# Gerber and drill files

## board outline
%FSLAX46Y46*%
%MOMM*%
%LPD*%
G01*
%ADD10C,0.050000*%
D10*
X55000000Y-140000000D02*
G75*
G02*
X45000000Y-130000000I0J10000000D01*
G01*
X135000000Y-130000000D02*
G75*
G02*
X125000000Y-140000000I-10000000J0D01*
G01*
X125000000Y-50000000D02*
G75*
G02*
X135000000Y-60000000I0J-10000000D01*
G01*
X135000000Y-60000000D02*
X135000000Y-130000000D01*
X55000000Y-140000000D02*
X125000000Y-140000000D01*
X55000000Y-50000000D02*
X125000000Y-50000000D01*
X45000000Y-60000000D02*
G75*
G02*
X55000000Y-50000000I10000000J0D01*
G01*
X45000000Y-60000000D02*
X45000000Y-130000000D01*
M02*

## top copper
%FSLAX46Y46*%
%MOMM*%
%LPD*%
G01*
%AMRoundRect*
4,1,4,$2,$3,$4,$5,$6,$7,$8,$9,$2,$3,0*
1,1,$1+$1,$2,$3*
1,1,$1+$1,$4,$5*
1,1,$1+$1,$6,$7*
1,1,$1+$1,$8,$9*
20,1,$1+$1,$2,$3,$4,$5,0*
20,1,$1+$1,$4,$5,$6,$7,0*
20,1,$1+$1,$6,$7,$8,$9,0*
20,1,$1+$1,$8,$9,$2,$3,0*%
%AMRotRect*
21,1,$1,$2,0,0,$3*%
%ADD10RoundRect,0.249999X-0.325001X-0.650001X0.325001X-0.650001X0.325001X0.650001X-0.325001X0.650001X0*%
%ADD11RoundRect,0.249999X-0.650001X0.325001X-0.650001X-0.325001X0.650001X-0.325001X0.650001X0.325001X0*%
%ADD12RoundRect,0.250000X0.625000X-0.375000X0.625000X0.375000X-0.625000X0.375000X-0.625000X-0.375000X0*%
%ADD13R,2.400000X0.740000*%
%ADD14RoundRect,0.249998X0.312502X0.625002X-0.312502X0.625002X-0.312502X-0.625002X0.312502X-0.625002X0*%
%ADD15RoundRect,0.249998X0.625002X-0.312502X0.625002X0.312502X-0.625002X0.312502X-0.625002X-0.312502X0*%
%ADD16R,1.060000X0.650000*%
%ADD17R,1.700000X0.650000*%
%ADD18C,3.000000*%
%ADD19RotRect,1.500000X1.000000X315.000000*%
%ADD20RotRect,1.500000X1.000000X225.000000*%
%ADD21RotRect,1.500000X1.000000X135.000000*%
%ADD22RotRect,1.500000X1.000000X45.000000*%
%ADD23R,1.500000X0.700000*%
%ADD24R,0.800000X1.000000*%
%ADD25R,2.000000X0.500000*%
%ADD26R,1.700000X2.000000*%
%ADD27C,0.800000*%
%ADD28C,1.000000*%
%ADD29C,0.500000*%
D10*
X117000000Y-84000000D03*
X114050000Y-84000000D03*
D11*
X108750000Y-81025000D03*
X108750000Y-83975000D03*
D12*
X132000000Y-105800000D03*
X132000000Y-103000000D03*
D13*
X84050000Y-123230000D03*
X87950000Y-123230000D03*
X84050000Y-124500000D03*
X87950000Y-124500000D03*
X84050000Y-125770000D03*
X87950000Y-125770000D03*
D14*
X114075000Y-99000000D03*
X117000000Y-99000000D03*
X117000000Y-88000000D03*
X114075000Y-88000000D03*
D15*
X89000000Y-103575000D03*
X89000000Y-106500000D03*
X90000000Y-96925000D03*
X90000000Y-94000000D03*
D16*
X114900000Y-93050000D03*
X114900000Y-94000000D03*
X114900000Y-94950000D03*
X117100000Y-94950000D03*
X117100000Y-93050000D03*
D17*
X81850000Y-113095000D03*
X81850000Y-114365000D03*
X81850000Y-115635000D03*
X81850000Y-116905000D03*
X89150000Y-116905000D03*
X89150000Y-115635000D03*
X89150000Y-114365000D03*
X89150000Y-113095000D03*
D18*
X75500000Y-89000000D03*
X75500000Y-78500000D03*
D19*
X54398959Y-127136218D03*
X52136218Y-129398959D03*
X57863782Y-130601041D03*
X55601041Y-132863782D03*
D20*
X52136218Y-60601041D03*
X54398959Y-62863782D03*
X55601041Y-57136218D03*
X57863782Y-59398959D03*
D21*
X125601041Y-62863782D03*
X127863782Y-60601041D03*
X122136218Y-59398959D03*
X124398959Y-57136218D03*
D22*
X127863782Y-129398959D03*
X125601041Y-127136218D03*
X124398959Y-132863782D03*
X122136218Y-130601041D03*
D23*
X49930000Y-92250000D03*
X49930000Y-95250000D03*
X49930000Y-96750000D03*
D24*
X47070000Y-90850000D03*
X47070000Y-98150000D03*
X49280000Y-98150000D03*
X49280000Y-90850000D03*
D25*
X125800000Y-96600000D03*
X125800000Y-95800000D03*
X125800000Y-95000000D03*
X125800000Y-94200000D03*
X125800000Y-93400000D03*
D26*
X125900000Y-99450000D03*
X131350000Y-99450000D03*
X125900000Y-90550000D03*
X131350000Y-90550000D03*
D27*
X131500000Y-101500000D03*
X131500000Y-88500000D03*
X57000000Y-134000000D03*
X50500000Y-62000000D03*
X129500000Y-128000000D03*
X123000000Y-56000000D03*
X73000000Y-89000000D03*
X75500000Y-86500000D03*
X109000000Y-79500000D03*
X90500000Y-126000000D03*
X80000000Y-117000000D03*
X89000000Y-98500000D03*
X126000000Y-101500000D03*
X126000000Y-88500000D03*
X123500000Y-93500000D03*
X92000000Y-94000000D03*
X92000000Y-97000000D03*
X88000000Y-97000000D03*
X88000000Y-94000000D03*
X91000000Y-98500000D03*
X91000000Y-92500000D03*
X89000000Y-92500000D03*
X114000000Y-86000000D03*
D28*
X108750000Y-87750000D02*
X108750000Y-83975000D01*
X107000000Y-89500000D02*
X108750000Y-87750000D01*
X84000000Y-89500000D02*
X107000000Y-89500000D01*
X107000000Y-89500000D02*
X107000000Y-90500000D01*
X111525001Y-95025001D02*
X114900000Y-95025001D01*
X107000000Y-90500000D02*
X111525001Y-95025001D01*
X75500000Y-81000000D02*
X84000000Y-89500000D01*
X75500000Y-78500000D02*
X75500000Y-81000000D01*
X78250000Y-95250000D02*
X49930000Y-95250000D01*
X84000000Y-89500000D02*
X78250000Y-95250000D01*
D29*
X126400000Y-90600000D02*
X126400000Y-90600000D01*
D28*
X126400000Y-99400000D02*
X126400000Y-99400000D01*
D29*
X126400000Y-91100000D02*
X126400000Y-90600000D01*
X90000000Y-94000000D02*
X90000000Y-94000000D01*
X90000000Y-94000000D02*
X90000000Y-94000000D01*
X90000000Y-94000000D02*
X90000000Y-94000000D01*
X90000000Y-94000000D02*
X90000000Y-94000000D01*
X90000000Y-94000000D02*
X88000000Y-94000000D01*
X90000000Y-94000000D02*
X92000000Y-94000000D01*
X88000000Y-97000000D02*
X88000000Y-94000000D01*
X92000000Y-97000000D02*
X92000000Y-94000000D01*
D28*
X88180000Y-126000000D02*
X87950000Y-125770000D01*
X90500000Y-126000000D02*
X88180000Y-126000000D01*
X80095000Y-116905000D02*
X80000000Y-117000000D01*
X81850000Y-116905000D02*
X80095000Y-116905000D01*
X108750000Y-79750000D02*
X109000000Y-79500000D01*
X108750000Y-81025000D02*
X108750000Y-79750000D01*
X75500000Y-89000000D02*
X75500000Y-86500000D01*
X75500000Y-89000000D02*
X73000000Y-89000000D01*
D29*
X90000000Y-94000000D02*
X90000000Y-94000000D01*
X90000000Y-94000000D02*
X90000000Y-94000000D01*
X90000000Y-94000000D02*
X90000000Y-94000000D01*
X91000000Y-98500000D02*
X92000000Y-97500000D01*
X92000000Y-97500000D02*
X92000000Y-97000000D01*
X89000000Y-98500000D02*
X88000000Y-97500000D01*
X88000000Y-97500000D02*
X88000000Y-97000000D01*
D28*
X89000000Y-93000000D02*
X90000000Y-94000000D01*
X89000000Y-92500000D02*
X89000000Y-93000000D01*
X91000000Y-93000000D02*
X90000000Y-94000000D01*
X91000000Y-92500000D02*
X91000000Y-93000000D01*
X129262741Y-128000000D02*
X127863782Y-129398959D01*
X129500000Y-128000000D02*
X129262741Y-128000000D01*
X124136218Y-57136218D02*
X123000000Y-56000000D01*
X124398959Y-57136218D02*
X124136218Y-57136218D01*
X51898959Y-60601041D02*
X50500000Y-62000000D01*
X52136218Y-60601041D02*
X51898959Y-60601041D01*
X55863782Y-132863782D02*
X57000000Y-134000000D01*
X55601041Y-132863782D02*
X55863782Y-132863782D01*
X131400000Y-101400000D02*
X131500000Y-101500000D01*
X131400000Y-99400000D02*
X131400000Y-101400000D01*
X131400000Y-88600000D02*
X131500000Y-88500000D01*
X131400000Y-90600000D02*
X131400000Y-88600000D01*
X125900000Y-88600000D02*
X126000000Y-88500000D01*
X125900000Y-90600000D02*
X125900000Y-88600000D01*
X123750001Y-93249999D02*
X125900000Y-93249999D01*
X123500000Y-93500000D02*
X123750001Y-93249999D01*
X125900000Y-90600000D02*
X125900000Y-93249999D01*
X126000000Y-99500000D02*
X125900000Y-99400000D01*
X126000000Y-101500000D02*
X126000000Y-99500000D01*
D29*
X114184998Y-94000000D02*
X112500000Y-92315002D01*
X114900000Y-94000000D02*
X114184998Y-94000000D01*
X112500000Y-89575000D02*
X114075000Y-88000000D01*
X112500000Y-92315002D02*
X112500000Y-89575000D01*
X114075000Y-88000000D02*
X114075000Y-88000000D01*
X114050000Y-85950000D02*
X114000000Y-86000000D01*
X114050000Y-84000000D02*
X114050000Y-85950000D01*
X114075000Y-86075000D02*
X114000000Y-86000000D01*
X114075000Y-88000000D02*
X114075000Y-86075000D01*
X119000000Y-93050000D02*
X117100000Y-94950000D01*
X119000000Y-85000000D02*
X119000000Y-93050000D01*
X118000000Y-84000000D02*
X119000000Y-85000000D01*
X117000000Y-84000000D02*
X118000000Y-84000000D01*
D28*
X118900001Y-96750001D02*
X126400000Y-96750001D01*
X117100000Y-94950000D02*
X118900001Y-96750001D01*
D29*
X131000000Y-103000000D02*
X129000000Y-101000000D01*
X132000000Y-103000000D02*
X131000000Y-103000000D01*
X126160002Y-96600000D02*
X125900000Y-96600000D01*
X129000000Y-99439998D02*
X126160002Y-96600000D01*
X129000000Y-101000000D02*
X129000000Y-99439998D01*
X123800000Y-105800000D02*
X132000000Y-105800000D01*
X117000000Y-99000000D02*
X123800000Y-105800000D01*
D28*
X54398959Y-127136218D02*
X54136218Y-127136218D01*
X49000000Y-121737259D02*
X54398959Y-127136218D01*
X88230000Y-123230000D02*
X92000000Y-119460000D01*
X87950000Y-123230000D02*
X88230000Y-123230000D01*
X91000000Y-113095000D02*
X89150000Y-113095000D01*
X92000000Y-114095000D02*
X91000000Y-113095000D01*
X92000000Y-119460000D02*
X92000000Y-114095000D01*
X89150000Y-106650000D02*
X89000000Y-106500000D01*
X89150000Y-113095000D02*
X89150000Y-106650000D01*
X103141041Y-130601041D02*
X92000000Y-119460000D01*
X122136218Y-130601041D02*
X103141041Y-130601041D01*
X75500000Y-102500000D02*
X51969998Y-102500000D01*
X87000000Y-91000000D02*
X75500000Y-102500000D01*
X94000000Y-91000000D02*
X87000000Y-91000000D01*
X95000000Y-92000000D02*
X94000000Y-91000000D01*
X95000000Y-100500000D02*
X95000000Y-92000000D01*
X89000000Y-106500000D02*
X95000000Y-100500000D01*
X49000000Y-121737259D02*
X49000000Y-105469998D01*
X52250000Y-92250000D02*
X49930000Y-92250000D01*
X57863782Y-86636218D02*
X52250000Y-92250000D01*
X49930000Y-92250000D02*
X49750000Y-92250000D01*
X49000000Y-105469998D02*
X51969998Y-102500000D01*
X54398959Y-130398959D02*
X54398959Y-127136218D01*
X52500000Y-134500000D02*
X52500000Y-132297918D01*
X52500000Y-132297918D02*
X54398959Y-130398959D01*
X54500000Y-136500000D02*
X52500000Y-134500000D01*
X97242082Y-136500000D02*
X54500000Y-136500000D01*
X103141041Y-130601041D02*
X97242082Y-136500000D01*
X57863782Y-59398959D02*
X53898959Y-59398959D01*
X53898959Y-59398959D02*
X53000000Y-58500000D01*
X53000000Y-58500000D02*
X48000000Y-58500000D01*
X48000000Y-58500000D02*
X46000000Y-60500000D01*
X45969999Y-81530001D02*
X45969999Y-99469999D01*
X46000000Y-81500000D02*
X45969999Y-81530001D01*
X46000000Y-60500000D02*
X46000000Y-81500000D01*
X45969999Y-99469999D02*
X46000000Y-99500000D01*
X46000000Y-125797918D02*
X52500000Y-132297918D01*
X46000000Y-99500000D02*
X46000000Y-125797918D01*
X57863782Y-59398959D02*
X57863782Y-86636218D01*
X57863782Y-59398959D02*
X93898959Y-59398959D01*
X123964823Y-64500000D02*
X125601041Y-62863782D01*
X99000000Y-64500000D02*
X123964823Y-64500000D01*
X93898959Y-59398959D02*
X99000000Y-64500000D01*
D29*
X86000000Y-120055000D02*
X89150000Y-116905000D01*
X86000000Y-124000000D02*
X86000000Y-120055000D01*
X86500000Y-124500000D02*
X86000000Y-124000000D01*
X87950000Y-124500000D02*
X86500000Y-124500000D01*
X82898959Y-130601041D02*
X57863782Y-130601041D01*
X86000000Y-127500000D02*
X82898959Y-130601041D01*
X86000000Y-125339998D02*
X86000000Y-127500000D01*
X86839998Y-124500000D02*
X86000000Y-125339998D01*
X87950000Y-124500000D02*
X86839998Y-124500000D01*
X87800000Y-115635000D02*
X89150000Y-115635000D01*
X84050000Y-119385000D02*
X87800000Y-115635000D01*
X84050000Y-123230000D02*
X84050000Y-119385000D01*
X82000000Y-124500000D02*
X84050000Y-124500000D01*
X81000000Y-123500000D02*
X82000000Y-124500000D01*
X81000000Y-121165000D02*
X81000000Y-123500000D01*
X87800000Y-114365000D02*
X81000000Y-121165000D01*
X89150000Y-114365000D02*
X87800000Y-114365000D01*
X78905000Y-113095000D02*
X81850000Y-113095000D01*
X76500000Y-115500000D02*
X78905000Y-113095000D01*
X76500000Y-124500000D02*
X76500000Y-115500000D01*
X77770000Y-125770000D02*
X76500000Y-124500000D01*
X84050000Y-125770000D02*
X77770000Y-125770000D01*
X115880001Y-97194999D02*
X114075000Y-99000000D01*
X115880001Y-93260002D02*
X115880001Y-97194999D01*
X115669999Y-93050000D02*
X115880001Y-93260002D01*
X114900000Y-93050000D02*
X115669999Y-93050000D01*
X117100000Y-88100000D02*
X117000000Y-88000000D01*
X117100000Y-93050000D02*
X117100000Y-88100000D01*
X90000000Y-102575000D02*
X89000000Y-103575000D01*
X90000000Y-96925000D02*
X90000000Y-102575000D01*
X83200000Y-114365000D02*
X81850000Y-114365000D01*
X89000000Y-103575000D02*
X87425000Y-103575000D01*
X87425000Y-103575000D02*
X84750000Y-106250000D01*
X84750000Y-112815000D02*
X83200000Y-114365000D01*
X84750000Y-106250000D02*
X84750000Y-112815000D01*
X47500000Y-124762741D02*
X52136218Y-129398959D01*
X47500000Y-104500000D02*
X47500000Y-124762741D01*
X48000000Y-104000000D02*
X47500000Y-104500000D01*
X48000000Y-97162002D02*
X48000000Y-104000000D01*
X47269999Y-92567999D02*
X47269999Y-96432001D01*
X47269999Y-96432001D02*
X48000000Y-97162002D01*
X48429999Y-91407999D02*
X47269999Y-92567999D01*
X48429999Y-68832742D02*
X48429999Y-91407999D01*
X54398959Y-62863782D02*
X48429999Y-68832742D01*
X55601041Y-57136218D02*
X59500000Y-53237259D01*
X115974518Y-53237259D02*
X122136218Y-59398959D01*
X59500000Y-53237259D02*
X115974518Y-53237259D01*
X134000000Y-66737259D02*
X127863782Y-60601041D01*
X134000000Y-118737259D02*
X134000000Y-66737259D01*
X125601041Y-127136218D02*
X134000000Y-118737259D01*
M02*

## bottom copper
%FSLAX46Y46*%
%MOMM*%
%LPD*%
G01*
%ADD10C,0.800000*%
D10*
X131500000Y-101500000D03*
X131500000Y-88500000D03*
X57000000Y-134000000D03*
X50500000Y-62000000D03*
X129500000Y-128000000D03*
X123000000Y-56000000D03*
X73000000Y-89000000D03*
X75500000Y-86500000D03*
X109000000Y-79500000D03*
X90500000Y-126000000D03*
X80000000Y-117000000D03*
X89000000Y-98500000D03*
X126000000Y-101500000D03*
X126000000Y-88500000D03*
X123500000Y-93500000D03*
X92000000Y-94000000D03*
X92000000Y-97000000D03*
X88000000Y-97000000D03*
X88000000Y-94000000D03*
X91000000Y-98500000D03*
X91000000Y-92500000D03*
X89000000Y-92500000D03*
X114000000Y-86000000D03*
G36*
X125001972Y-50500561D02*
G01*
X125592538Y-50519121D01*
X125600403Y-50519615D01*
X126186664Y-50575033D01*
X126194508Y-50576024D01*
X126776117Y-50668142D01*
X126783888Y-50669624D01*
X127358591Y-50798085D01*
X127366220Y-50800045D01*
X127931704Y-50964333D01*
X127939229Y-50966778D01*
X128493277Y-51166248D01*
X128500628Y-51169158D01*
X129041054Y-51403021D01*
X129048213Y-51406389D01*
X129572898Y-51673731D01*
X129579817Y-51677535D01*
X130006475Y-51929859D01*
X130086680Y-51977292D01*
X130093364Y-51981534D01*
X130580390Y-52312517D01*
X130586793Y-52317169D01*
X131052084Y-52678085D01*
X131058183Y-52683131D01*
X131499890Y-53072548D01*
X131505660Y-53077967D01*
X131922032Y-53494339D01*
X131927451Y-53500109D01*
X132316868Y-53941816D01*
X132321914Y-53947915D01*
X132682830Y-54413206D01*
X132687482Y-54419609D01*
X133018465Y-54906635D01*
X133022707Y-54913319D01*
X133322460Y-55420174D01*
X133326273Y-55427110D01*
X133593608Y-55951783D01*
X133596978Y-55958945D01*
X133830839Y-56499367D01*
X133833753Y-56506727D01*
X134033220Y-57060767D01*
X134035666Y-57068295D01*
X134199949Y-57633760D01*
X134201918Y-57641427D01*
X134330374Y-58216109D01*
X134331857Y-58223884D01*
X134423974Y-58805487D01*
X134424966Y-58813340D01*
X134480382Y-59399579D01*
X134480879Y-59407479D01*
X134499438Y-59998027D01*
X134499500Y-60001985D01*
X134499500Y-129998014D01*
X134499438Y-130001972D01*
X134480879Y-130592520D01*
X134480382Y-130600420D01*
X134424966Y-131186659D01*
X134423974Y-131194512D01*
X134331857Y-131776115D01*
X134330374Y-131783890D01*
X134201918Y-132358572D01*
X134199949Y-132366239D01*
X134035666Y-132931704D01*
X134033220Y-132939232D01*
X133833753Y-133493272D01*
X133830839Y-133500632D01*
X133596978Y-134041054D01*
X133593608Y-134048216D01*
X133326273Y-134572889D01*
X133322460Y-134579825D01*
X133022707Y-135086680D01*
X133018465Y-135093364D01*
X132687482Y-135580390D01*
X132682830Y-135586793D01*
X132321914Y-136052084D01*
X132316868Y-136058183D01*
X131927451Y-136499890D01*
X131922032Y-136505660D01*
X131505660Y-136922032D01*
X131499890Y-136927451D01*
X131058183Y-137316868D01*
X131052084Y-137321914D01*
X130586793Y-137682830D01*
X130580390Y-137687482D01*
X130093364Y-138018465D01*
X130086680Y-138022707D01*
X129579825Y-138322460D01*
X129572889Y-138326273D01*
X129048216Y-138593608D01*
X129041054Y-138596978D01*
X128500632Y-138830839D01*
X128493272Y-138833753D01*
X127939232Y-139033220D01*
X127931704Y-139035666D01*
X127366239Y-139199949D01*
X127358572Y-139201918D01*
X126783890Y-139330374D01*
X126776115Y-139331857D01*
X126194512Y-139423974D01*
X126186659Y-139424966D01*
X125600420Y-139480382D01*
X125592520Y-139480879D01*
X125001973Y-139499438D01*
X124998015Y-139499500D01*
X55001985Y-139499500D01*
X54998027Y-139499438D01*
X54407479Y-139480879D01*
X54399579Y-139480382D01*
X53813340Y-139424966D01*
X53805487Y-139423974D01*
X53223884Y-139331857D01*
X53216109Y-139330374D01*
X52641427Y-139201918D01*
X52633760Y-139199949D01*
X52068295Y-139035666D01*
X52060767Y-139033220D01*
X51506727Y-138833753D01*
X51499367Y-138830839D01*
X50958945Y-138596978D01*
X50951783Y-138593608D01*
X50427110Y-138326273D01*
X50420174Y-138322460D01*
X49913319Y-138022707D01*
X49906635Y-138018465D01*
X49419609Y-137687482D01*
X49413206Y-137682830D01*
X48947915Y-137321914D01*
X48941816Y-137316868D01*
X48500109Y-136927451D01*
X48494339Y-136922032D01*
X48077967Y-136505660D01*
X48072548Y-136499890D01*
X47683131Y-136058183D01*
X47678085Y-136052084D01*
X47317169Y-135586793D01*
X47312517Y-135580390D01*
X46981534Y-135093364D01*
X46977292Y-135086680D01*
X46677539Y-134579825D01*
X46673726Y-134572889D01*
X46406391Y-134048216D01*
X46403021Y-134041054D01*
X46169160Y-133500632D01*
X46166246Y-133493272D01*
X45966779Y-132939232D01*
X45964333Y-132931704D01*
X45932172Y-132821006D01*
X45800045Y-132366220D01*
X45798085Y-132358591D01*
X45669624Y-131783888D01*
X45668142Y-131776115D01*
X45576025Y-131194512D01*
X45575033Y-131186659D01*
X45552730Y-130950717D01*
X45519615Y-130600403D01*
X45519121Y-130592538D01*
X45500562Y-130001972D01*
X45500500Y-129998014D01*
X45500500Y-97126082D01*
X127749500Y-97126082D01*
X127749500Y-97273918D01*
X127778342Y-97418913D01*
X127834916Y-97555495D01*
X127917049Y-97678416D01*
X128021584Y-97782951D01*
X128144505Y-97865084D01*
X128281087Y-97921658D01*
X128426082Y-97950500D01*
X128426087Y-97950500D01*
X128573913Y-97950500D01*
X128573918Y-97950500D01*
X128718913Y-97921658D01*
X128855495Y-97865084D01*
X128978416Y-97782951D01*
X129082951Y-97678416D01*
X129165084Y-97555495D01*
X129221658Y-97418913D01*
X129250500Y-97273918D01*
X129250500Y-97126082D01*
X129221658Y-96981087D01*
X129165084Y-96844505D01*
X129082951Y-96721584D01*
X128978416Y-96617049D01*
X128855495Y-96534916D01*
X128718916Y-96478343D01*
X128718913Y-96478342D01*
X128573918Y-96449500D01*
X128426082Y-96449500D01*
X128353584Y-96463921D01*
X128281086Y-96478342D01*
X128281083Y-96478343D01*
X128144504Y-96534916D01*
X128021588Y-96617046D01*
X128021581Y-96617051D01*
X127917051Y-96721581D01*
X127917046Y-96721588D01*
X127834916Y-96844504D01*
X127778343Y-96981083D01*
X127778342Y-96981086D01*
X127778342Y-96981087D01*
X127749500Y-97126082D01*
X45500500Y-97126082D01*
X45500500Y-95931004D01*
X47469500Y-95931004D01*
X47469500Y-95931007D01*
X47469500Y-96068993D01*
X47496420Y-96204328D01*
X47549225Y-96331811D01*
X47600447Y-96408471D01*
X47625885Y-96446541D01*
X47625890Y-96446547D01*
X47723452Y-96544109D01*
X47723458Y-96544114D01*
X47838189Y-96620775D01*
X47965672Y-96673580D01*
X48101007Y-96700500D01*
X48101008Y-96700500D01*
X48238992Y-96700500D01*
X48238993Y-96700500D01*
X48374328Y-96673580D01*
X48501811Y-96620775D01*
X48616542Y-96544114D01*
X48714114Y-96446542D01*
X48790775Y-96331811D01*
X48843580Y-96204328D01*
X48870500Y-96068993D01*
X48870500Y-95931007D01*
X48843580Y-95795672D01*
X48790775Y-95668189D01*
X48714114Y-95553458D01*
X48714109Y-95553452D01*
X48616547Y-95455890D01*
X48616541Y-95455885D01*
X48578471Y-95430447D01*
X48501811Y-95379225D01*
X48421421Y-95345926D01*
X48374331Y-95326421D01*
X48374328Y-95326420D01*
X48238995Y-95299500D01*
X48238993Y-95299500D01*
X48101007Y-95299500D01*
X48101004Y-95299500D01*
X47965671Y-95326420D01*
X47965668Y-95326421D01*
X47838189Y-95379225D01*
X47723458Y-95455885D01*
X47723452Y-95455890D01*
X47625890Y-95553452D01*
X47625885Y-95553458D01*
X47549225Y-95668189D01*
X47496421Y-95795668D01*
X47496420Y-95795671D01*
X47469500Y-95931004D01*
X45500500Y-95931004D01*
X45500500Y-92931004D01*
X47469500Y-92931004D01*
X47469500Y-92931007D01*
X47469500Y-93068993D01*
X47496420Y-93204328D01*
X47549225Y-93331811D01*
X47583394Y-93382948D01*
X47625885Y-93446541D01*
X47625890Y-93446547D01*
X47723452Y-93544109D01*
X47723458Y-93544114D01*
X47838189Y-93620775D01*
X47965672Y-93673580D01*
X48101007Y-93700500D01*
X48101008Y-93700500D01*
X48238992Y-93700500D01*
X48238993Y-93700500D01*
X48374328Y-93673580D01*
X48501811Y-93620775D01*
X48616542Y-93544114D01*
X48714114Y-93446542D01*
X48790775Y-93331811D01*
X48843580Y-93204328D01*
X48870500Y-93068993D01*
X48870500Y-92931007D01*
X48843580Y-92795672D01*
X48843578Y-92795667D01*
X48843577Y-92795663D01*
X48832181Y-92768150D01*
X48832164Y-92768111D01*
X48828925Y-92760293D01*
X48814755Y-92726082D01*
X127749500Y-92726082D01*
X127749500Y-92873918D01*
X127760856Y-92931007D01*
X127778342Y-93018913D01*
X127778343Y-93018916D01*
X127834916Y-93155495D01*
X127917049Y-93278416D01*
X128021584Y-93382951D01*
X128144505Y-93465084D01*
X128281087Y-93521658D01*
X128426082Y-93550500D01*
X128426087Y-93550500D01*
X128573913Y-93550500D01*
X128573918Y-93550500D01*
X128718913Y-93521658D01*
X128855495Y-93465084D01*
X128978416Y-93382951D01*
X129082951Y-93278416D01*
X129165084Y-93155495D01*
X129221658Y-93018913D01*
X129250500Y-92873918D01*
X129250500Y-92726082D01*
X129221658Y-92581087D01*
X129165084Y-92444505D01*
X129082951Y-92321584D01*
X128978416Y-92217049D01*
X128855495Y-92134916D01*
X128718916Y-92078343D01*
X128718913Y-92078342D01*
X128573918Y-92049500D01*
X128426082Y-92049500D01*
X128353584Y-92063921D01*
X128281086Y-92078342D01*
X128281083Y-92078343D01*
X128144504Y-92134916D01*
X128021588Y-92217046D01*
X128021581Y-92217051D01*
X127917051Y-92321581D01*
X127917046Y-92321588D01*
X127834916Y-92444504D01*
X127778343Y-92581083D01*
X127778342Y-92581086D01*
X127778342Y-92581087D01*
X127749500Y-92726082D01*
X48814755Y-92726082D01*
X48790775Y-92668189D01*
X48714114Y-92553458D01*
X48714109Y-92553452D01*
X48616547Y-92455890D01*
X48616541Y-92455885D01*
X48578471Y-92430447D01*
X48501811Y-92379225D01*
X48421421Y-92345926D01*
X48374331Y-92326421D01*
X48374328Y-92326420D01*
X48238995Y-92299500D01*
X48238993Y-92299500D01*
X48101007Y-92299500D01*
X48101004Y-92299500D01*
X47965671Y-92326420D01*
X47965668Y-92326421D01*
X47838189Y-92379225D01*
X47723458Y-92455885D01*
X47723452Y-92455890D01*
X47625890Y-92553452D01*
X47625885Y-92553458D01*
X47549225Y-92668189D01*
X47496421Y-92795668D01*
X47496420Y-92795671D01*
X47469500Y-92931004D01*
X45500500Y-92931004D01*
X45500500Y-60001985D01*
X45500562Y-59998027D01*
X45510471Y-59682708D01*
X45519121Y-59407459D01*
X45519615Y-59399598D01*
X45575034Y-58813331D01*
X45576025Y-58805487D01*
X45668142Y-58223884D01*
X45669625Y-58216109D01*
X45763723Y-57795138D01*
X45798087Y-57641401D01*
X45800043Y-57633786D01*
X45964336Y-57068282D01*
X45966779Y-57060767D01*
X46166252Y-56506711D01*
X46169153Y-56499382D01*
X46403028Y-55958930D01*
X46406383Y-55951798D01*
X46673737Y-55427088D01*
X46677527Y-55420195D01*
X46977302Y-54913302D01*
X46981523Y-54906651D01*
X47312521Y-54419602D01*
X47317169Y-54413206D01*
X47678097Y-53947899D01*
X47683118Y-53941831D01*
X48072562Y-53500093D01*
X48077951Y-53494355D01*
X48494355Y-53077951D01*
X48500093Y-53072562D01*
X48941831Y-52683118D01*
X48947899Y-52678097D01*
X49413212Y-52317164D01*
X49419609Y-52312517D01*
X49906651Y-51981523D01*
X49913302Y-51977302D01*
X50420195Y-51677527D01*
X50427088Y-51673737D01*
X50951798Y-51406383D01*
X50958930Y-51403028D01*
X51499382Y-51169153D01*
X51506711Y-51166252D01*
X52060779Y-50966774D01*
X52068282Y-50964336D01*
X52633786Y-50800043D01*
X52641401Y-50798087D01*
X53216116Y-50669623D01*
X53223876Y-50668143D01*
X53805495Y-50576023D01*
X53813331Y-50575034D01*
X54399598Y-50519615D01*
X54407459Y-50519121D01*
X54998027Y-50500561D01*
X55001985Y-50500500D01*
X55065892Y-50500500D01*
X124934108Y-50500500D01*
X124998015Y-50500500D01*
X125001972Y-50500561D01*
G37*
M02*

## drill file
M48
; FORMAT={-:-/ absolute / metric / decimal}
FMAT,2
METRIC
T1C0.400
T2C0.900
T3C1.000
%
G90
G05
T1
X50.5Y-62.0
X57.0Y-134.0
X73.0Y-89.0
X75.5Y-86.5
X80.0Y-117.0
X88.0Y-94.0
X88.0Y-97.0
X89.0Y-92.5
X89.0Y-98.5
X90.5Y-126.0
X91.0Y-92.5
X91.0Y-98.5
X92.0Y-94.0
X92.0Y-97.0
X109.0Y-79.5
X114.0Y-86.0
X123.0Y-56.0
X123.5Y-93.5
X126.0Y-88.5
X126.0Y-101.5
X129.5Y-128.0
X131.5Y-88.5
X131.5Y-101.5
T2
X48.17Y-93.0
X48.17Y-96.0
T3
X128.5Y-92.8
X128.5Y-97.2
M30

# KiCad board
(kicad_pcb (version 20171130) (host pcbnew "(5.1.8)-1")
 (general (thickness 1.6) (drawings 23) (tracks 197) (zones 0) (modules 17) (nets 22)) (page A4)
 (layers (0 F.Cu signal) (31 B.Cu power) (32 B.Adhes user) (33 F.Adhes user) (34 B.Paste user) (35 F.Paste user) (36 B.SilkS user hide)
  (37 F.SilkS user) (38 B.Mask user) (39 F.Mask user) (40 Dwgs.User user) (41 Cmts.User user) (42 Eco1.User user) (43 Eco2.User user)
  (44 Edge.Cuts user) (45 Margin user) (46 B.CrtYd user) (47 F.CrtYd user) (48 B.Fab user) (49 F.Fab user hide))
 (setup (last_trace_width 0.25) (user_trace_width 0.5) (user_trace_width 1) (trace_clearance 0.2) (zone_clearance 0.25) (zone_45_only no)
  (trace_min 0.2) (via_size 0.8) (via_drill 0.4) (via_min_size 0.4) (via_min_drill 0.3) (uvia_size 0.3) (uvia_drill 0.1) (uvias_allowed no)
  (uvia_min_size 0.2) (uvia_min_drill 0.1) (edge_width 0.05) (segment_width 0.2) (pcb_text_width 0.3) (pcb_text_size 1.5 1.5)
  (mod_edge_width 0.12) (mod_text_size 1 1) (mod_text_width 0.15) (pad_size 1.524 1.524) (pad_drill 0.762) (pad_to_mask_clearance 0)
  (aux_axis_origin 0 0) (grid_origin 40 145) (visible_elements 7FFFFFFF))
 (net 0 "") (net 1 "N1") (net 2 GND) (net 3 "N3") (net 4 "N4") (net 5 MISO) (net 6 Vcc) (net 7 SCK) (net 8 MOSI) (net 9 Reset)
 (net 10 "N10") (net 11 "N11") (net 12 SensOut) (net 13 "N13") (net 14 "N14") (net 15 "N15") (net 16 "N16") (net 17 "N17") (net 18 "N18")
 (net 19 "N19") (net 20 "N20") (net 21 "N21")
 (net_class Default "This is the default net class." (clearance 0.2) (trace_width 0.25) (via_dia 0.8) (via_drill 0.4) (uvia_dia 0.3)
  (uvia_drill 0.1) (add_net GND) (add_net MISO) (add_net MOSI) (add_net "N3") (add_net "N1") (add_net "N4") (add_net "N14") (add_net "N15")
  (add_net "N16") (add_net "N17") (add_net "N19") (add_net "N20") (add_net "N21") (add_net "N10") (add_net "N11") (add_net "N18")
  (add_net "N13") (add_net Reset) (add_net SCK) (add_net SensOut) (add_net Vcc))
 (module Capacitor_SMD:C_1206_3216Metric (layer F.Cu) (at 115.525 84)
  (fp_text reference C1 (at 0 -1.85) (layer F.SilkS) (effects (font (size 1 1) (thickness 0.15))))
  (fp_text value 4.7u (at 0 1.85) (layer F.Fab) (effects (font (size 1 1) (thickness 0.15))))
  (pad 2 smd roundrect (at 1.475 0) (size 1.15 1.8) (layers F.Cu F.Paste F.Mask) (roundrect_rratio 0.2173904347826087) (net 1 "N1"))
  (pad 1 smd roundrect (at -1.475 0) (size 1.15 1.8) (layers F.Cu F.Paste F.Mask) (roundrect_rratio 0.2173904347826087) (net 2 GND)))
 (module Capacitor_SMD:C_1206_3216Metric (layer F.Cu) (at 108.75 82.5 270)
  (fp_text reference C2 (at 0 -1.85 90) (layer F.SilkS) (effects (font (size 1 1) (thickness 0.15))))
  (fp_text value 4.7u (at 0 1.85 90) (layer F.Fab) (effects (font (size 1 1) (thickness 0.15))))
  (pad 1 smd roundrect (at -1.475 0 270) (size 1.15 1.8) (layers F.Cu F.Paste F.Mask) (roundrect_rratio 0.2173904347826087) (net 2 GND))
  (pad 2 smd roundrect (at 1.475 0 270) (size 1.15 1.8) (layers F.Cu F.Paste F.Mask) (roundrect_rratio 0.2173904347826087) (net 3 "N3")))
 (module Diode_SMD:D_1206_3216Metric (layer F.Cu) (at 132 104.4 90)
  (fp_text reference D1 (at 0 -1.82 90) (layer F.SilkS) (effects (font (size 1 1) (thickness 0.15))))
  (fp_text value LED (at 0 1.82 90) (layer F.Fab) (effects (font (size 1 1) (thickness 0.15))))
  (pad 1 smd roundrect (at -1.4 0 90) (size 1.25 1.75) (layers F.Cu F.Paste F.Mask) (roundrect_rratio 0.2) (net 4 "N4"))
  (pad 2 smd roundrect (at 1.4 0 90) (size 1.25 1.75) (layers F.Cu F.Paste F.Mask) (roundrect_rratio 0.2) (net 1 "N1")))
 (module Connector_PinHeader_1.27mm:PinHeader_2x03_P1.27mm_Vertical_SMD (layer F.Cu) (at 86 124.5)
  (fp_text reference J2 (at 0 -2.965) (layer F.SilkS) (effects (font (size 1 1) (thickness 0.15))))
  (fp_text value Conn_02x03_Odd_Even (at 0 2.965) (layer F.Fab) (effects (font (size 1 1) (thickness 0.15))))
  (pad 1 smd rect (at -1.95 -1.27) (size 2.4 0.74) (layers F.Cu F.Paste F.Mask) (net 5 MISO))
  (pad 2 smd rect (at 1.95 -1.27) (size 2.4 0.74) (layers F.Cu F.Paste F.Mask) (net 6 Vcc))
  (pad 3 smd rect (at -1.95 0) (size 2.4 0.74) (layers F.Cu F.Paste F.Mask) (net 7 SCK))
  (pad 4 smd rect (at 1.95 0) (size 2.4 0.74) (layers F.Cu F.Paste F.Mask) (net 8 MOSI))
  (pad 5 smd rect (at -1.95 1.27) (size 2.4 0.74) (layers F.Cu F.Paste F.Mask) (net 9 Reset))
  (pad 6 smd rect (at 1.95 1.27) (size 2.4 0.74) (layers F.Cu F.Paste F.Mask) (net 2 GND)))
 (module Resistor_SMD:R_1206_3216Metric (layer F.Cu) (at 115.5375 99 180)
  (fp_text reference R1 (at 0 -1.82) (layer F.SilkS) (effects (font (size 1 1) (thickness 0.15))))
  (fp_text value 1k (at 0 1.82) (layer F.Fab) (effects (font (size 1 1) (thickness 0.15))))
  (pad 2 smd roundrect (at 1.4625 0 180) (size 1.125 1.75) (layers F.Cu F.Paste F.Mask) (roundrect_rratio 0.2222204444444444) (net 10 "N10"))
  (pad 1 smd roundrect (at -1.4625 0 180) (size 1.125 1.75) (layers F.Cu F.Paste F.Mask) (roundrect_rratio 0.2222204444444444) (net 4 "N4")))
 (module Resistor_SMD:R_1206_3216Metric (layer F.Cu) (at 115.5375 88 180)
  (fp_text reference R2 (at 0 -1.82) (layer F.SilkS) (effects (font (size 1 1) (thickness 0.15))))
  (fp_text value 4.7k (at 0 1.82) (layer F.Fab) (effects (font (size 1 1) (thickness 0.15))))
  (pad 1 smd roundrect (at -1.4625 0 180) (size 1.125 1.75) (layers F.Cu F.Paste F.Mask) (roundrect_rratio 0.2222204444444444)
   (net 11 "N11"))
  (pad 2 smd roundrect (at 1.4625 0 180) (size 1.125 1.75) (layers F.Cu F.Paste F.Mask) (roundrect_rratio 0.2222204444444444) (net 2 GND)))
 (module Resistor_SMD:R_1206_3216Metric (layer F.Cu) (at 89 105.0375 90)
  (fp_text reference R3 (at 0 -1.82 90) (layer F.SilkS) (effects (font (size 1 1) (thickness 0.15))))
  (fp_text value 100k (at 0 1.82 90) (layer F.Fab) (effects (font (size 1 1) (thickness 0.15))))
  (pad 2 smd roundrect (at 1.4625 0 90) (size 1.125 1.75) (layers F.Cu F.Paste F.Mask) (roundrect_rratio 0.2222204444444444)
   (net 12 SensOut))
  (pad 1 smd roundrect (at -1.4625 0 90) (size 1.125 1.75) (layers F.Cu F.Paste F.Mask) (roundrect_rratio 0.2222204444444444) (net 6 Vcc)))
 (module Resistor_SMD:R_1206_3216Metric (layer F.Cu) (at 90 95.4625 90)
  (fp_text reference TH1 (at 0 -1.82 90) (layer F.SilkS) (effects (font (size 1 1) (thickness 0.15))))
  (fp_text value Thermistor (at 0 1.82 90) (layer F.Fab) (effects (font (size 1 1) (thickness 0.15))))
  (pad 1 smd roundrect (at -1.4625 0 90) (size 1.125 1.75) (layers F.Cu F.Paste F.Mask) (roundrect_rratio 0.2222204444444444)
   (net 12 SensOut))
  (pad 2 smd roundrect (at 1.4625 0 90) (size 1.125 1.75) (layers F.Cu F.Paste F.Mask) (roundrect_rratio 0.2222204444444444) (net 2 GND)))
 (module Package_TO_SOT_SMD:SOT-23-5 (layer F.Cu) (at 116 94)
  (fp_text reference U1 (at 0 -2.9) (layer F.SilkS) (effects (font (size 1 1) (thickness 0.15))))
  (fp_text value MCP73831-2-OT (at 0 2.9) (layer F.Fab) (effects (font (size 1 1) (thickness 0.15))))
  (pad 1 smd rect (at -1.1 -0.95) (size 1.06 0.65) (layers F.Cu F.Paste F.Mask) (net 10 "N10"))
  (pad 2 smd rect (at -1.1 0) (size 1.06 0.65) (layers F.Cu F.Paste F.Mask) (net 2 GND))
  (pad 3 smd rect (at -1.1 0.95) (size 1.06 0.65) (layers F.Cu F.Paste F.Mask) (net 3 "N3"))
  (pad 4 smd rect (at 1.1 0.95) (size 1.06 0.65) (layers F.Cu F.Paste F.Mask) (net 1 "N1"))
  (pad 5 smd rect (at 1.1 -0.95) (size 1.06 0.65) (layers F.Cu F.Paste F.Mask) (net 11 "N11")))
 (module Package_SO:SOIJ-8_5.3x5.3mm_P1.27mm (layer F.Cu) (at 85.5 115)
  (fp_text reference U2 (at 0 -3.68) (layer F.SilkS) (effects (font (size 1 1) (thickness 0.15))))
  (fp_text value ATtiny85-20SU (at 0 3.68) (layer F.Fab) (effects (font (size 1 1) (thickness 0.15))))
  (pad 1 smd rect (at -3.65 -1.905) (size 1.7 0.65) (layers F.Cu F.Paste F.Mask) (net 9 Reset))
  (pad 2 smd rect (at -3.65 -0.635) (size 1.7 0.65) (layers F.Cu F.Paste F.Mask) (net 12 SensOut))
  (pad 3 smd rect (at -3.65 0.635) (size 1.7 0.65) (layers F.Cu F.Paste F.Mask) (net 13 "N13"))
  (pad 4 smd rect (at -3.65 1.905) (size 1.7 0.65) (layers F.Cu F.Paste F.Mask) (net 2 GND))
  (pad 5 smd rect (at 3.65 1.905) (size 1.7 0.65) (layers F.Cu F.Paste F.Mask) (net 8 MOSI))
  (pad 6 smd rect (at 3.65 0.635) (size 1.7 0.65) (layers F.Cu F.Paste F.Mask) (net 5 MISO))
  (pad 7 smd rect (at 3.65 -0.635) (size 1.7 0.65) (layers F.Cu F.Paste F.Mask) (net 7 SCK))
  (pad 8 smd rect (at 3.65 -1.905) (size 1.7 0.65) (layers F.Cu F.Paste F.Mask) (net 6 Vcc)))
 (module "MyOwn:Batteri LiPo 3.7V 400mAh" (layer F.Cu) (at 93.5 75 270)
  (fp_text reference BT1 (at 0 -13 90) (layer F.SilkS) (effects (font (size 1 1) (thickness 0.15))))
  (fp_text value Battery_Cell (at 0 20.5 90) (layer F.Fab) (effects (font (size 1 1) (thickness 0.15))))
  (pad 2 smd circle (at 14 18 270) (size 3 3) (layers F.Cu F.Paste F.Mask) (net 2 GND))
  (pad 1 smd circle (at 3.5 18 270) (size 3 3) (layers F.Cu F.Paste F.Mask) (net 3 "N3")))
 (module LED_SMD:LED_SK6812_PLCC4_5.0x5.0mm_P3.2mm (layer F.Cu) (at 55 130 315)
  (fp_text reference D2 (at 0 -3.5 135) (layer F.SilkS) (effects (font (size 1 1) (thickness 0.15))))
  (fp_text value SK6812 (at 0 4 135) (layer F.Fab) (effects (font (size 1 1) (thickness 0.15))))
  (pad 3 smd rect (at -2.45 -1.6 315) (size 1.5 1) (layers F.Cu F.Paste F.Mask) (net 6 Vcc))
  (pad 4 smd rect (at -2.45 1.6 315) (size 1.5 1) (layers F.Cu F.Paste F.Mask) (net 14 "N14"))
  (pad 2 smd rect (at 2.45 -1.6 315) (size 1.5 1) (layers F.Cu F.Paste F.Mask) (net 8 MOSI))
  (pad 1 smd rect (at 2.45 1.6 315) (size 1.5 1) (layers F.Cu F.Paste F.Mask) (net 2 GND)))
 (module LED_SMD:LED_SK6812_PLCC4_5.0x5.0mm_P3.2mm (layer F.Cu) (at 55 60 225)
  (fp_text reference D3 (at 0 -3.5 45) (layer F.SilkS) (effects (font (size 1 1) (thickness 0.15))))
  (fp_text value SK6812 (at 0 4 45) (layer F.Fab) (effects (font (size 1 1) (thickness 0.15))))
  (pad 1 smd rect (at 2.45 1.6 225) (size 1.5 1) (layers F.Cu F.Paste F.Mask) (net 2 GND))
  (pad 2 smd rect (at 2.45 -1.6 225) (size 1.5 1) (layers F.Cu F.Paste F.Mask) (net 14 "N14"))
  (pad 4 smd rect (at -2.45 1.6 225) (size 1.5 1) (layers F.Cu F.Paste F.Mask) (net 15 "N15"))
  (pad 3 smd rect (at -2.45 -1.6 225) (size 1.5 1) (layers F.Cu F.Paste F.Mask) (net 6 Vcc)))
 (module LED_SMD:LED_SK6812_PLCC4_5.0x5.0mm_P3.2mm (layer F.Cu) (at 125 60 135)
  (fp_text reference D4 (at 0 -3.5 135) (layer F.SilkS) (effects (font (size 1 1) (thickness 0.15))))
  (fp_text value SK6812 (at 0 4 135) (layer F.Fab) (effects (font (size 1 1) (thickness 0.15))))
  (pad 3 smd rect (at -2.45 -1.6 135) (size 1.5 1) (layers F.Cu F.Paste F.Mask) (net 6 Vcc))
  (pad 4 smd rect (at -2.45 1.6 135) (size 1.5 1) (layers F.Cu F.Paste F.Mask) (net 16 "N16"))
  (pad 2 smd rect (at 2.45 -1.6 135) (size 1.5 1) (layers F.Cu F.Paste F.Mask) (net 15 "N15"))
  (pad 1 smd rect (at 2.45 1.6 135) (size 1.5 1) (layers F.Cu F.Paste F.Mask) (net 2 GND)))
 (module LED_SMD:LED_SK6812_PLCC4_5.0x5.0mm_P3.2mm (layer F.Cu) (at 125 130 45)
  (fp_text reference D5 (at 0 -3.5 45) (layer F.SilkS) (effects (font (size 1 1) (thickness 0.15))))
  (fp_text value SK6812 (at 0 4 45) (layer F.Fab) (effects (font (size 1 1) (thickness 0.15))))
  (pad 1 smd rect (at 2.45 1.6 45) (size 1.5 1) (layers F.Cu F.Paste F.Mask) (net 2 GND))
  (pad 2 smd rect (at 2.45 -1.6 45) (size 1.5 1) (layers F.Cu F.Paste F.Mask) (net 16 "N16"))
  (pad 4 smd rect (at -2.45 1.6 45) (size 1.5 1) (layers F.Cu F.Paste F.Mask) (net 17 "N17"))
  (pad 3 smd rect (at -2.45 -1.6 45) (size 1.5 1) (layers F.Cu F.Paste F.Mask) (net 6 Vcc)))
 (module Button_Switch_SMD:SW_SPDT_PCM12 (layer F.Cu) (at 48.5 94.5 270)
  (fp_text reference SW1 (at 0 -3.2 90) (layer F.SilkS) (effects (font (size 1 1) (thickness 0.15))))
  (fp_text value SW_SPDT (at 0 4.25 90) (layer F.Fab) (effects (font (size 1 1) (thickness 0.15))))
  (pad "" np_thru_hole circle (at -1.5 0.33 270) (size 0.9 0.9) (drill 0.9) (layers *.Cu *.Mask))
  (pad "" np_thru_hole circle (at 1.5 0.33 270) (size 0.9 0.9) (drill 0.9) (layers *.Cu *.Mask))
  (pad 1 smd rect (at -2.25 -1.43 270) (size 0.7 1.5) (layers F.Cu F.Paste F.Mask) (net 6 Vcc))
  (pad 2 smd rect (at 0.75 -1.43 270) (size 0.7 1.5) (layers F.Cu F.Paste F.Mask) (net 3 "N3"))
  (pad 3 smd rect (at 2.25 -1.43 270) (size 0.7 1.5) (layers F.Cu F.Paste F.Mask) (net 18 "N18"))
  (pad "" smd rect (at -3.65 1.43 270) (size 1 0.8) (layers F.Cu F.Paste F.Mask))
  (pad "" smd rect (at 3.65 1.43 270) (size 1 0.8) (layers F.Cu F.Paste F.Mask))
  (pad "" smd rect (at 3.65 -0.78 270) (size 1 0.8) (layers F.Cu F.Paste F.Mask))
  (pad "" smd rect (at -3.65 -0.78 270) (size 1 0.8) (layers F.Cu F.Paste F.Mask)))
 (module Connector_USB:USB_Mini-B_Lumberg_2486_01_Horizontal (layer F.Cu) (at 128.5 95 90)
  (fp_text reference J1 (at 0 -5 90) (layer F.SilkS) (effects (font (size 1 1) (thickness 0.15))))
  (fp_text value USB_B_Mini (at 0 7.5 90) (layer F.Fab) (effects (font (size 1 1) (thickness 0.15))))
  (pad 1 smd rect (at -1.6 -2.7 90) (size 0.5 2) (layers F.Cu F.Paste F.Mask) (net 1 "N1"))
  (pad 2 smd rect (at -0.8 -2.7 90) (size 0.5 2) (layers F.Cu F.Paste F.Mask) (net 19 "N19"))
  (pad 3 smd rect (at 0 -2.7 90) (size 0.5 2) (layers F.Cu F.Paste F.Mask) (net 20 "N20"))
  (pad 4 smd rect (at 0.8 -2.7 90) (size 0.5 2) (layers F.Cu F.Paste F.Mask) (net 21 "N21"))
  (pad 5 smd rect (at 1.6 -2.7 90) (size 0.5 2) (layers F.Cu F.Paste F.Mask) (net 2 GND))
  (pad 6 smd rect (at -4.45 -2.6 90) (size 2 1.7) (layers F.Cu F.Paste F.Mask) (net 2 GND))
  (pad 6 smd rect (at -4.45 2.85 90) (size 2 1.7) (layers F.Cu F.Paste F.Mask) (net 2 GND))
  (pad 6 smd rect (at 4.45 -2.6 90) (size 2 1.7) (layers F.Cu F.Paste F.Mask) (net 2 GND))
  (pad 6 smd rect (at 4.45 2.85 90) (size 2 1.7) (layers F.Cu F.Paste F.Mask) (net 2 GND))
  (pad "" np_thru_hole circle (at -2.2 0 90) (size 1 1) (drill 1) (layers *.Cu *.Mask))
  (pad "" np_thru_hole circle (at 2.2 0 90) (size 1 1) (drill 1) (layers *.Cu *.Mask)))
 (gr_arc (start 55 130) (end 45 130) (angle -90) (layer Edge.Cuts) (width 0.05))
 (gr_arc (start 125 130) (end 125 140) (angle -90) (layer Edge.Cuts) (width 0.05))
 (gr_arc (start 125 60) (end 135 60) (angle -90) (layer Edge.Cuts) (width 0.05))
 (gr_line (start 135 60) (end 135 130) (layer Edge.Cuts) (width 0.05))
 (gr_line (start 55 140) (end 125 140) (layer Edge.Cuts) (width 0.05))
 (gr_line (start 55 50) (end 125 50) (layer Edge.Cuts) (width 0.05))
 (gr_arc (start 55 60) (end 55 50) (angle -90) (layer Edge.Cuts) (width 0.05))
 (gr_line (start 45 60) (end 45 130) (layer Edge.Cuts) (width 0.05))
 (segment (start 108.75 87.75) (end 108.75 83.975) (width 1) (layer F.Cu) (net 3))
 (segment (start 107 89.5) (end 108.75 87.75) (width 1) (layer F.Cu) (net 3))
 (segment (start 84 89.5) (end 107 89.5) (width 1) (layer F.Cu) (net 3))
 (segment (start 107 89.5) (end 107 90.5) (width 1) (layer F.Cu) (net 3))
 (segment (start 111.525001 95.025001) (end 114.9 95.025001) (width 1) (layer F.Cu) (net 3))
 (segment (start 107 90.5) (end 111.525001 95.025001) (width 1) (layer F.Cu) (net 3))
 (segment (start 75.5 81) (end 84 89.5) (width 1) (layer F.Cu) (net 3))
 (segment (start 75.5 78.5) (end 75.5 81) (width 1) (layer F.Cu) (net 3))
 (segment (start 78.25 95.25) (end 49.93 95.25) (width 1) (layer F.Cu) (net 3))
 (segment (start 84 89.5) (end 78.25 95.25) (width 1) (layer F.Cu) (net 3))
 (via (at 131.5 101.5) (size 0.8) (drill 0.4) (layers F.Cu B.Cu) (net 2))
 (via (at 131.5 88.5) (size 0.8) (drill 0.4) (layers F.Cu B.Cu) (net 2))
 (via (at 57 134) (size 0.8) (drill 0.4) (layers F.Cu B.Cu) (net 2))
 (via (at 50.5 62) (size 0.8) (drill 0.4) (layers F.Cu B.Cu) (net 2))
 (via (at 129.5 128) (size 0.8) (drill 0.4) (layers F.Cu B.Cu) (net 2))
 (via (at 123 56) (size 0.8) (drill 0.4) (layers F.Cu B.Cu) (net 2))
 (via (at 73 89) (size 0.8) (drill 0.4) (layers F.Cu B.Cu) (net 2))
 (via (at 75.5 86.5) (size 0.8) (drill 0.4) (layers F.Cu B.Cu) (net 2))
 (via (at 109 79.5) (size 0.8) (drill 0.4) (layers F.Cu B.Cu) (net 2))
 (via (at 90.5 126) (size 0.8) (drill 0.4) (layers F.Cu B.Cu) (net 2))
 (via (at 80 117) (size 0.8) (drill 0.4) (layers F.Cu B.Cu) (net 2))
 (via (at 89 98.5) (size 0.8) (drill 0.4) (layers F.Cu B.Cu) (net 2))
 (via (at 126 101.5) (size 0.8) (drill 0.4) (layers F.Cu B.Cu) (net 2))
 (segment (start 126.4 90.6) (end 126.4 90.6) (width 0.5) (layer F.Cu) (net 2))
 (via (at 126 88.5) (size 0.8) (drill 0.4) (layers F.Cu B.Cu) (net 2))
 (segment (start 126.4 99.4) (end 126.4 99.4) (width 1) (layer F.Cu) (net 2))
 (segment (start 126.4 91.1) (end 126.4 90.6) (width 0.5) (layer F.Cu) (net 2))
 (via (at 123.5 93.5) (size 0.8) (drill 0.4) (layers F.Cu B.Cu) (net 2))
 (segment (start 90 94) (end 90 94) (width 0.5) (layer F.Cu) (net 2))
 (segment (start 90 94) (end 90 94) (width 0.5) (layer F.Cu) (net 2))
 (via (at 92 94) (size 0.8) (drill 0.4) (layers F.Cu B.Cu) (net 2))
 (segment (start 90 94) (end 90 94) (width 0.5) (layer F.Cu) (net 2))
 (via (at 92 97) (size 0.8) (drill 0.4) (layers F.Cu B.Cu) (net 2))
 (segment (start 90 94) (end 90 94) (width 0.5) (layer F.Cu) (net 2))
 (via (at 88 97) (size 0.8) (drill 0.4) (layers F.Cu B.Cu) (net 2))
 (via (at 88 94) (size 0.8) (drill 0.4) (layers F.Cu B.Cu) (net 2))
 (segment (start 90 94) (end 88 94) (width 0.5) (layer F.Cu) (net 2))
 (segment (start 90 94) (end 92 94) (width 0.5) (layer F.Cu) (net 2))
 (segment (start 88 97) (end 88 94) (width 0.5) (layer F.Cu) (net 2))
 (segment (start 92 97) (end 92 94) (width 0.5) (layer F.Cu) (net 2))
 (segment (start 88.18 126) (end 87.95 125.77) (width 1) (layer F.Cu) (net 2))
 (segment (start 90.5 126) (end 88.18 126) (width 1) (layer F.Cu) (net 2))
 (segment (start 80.095 116.905) (end 80 117) (width 1) (layer F.Cu) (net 2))
 (segment (start 81.85 116.905) (end 80.095 116.905) (width 1) (layer F.Cu) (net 2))
 (segment (start 108.75 79.75) (end 109 79.5) (width 1) (layer F.Cu) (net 2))
 (segment (start 108.75 81.025) (end 108.75 79.75) (width 1) (layer F.Cu) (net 2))
 (segment (start 75.5 89) (end 75.5 86.5) (width 1) (layer F.Cu) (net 2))
 (segment (start 75.5 89) (end 73 89) (width 1) (layer F.Cu) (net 2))
 (segment (start 90 94) (end 90 94) (width 0.5) (layer F.Cu) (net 2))
 (via (at 91 98.5) (size 0.8) (drill 0.4) (layers F.Cu B.Cu) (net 2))
 (segment (start 90 94) (end 90 94) (width 0.5) (layer F.Cu) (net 2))
 (via (at 91 92.5) (size 0.8) (drill 0.4) (layers F.Cu B.Cu) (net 2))
 (segment (start 90 94) (end 90 94) (width 0.5) (layer F.Cu) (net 2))
 (via (at 89 92.5) (size 0.8) (drill 0.4) (layers F.Cu B.Cu) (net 2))
 (segment (start 91 98.5) (end 92 97.5) (width 0.5) (layer F.Cu) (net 2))
 (segment (start 92 97.5) (end 92 97) (width 0.5) (layer F.Cu) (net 2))
 (segment (start 89 98.5) (end 88 97.5) (width 0.5) (layer F.Cu) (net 2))
 (segment (start 88 97.5) (end 88 97) (width 0.5) (layer F.Cu) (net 2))
 (segment (start 89 93) (end 90 94) (width 1) (layer F.Cu) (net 2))
 (segment (start 89 92.5) (end 89 93) (width 1) (layer F.Cu) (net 2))
 (segment (start 91 93) (end 90 94) (width 1) (layer F.Cu) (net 2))
 (segment (start 91 92.5) (end 91 93) (width 1) (layer F.Cu) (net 2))
 (segment (start 129.262741 128) (end 127.863782 129.398959) (width 1) (layer F.Cu) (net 2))
 (segment (start 129.5 128) (end 129.262741 128) (width 1) (layer F.Cu) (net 2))
 (segment (start 124.136218 57.136218) (end 123 56) (width 1) (layer F.Cu) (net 2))
 (segment (start 124.398959 57.136218) (end 124.136218 57.136218) (width 1) (layer F.Cu) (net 2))
 (segment (start 51.898959 60.601041) (end 50.5 62) (width 1) (layer F.Cu) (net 2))
 (segment (start 52.136218 60.601041) (end 51.898959 60.601041) (width 1) (layer F.Cu) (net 2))
 (segment (start 55.863782 132.863782) (end 57 134) (width 1) (layer F.Cu) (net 2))
 (segment (start 55.601041 132.863782) (end 55.863782 132.863782) (width 1) (layer F.Cu) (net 2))
 (segment (start 131.4 101.4) (end 131.5 101.5) (width 1) (layer F.Cu) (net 2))
 (segment (start 131.4 99.4) (end 131.4 101.4) (width 1) (layer F.Cu) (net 2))
 (segment (start 131.4 88.6) (end 131.5 88.5) (width 1) (layer F.Cu) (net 2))
 (segment (start 131.4 90.6) (end 131.4 88.6) (width 1) (layer F.Cu) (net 2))
 (segment (start 125.9 88.6) (end 126 88.5) (width 1) (layer F.Cu) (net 2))
 (segment (start 125.9 90.6) (end 125.9 88.6) (width 1) (layer F.Cu) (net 2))
 (segment (start 123.750001 93.249999) (end 125.9 93.249999) (width 1) (layer F.Cu) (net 2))
 (segment (start 123.5 93.5) (end 123.750001 93.249999) (width 1) (layer F.Cu) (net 2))
 (segment (start 125.9 90.6) (end 125.9 93.249999) (width 1) (layer F.Cu) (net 2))
 (segment (start 126 99.5) (end 125.9 99.4) (width 1) (layer F.Cu) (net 2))
 (segment (start 126 101.5) (end 126 99.5) (width 1) (layer F.Cu) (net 2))
 (segment (start 114.184998 94) (end 112.5 92.315002) (width 0.5) (layer F.Cu) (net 2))
 (segment (start 114.9 94) (end 114.184998 94) (width 0.5) (layer F.Cu) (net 2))
 (segment (start 112.5 89.575) (end 114.075 88) (width 0.5) (layer F.Cu) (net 2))
 (segment (start 112.5 92.315002) (end 112.5 89.575) (width 0.5) (layer F.Cu) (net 2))
 (segment (start 114.075 88) (end 114.075 88) (width 0.5) (layer F.Cu) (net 2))
 (via (at 114 86) (size 0.8) (drill 0.4) (layers F.Cu B.Cu) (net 2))
 (segment (start 114.05 85.95) (end 114 86) (width 0.5) (layer F.Cu) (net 2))
 (segment (start 114.05 84) (end 114.05 85.95) (width 0.5) (layer F.Cu) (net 2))
 (segment (start 114.075 86.075) (end 114 86) (width 0.5) (layer F.Cu) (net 2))
 (segment (start 114.075 88) (end 114.075 86.075) (width 0.5) (layer F.Cu) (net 2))
 (segment (start 119 93.05) (end 117.1 94.95) (width 0.5) (layer F.Cu) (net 1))
 (segment (start 119 85) (end 119 93.05) (width 0.5) (layer F.Cu) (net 1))
 (segment (start 118 84) (end 119 85) (width 0.5) (layer F.Cu) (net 1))
 (segment (start 117 84) (end 118 84) (width 0.5) (layer F.Cu) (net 1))
 (segment (start 118.900001 96.750001) (end 126.4 96.750001) (width 1) (layer F.Cu) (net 1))
 (segment (start 117.1 94.95) (end 118.900001 96.750001) (width 1) (layer F.Cu) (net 1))
 (segment (start 131 103) (end 129 101) (width 0.5) (layer F.Cu) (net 1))
 (segment (start 132 103) (end 131 103) (width 0.5) (layer F.Cu) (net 1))
 (segment (start 126.160002 96.6) (end 125.9 96.6) (width 0.5) (layer F.Cu) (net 1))
 (segment (start 129 99.439998) (end 126.160002 96.6) (width 0.5) (layer F.Cu) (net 1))
 (segment (start 129 101) (end 129 99.439998) (width 0.5) (layer F.Cu) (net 1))
 (segment (start 123.8 105.8) (end 132 105.8) (width 0.5) (layer F.Cu) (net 4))
 (segment (start 117 99) (end 123.8 105.8) (width 0.5) (layer F.Cu) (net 4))
 (segment (start 54.398959 127.136218) (end 54.136218 127.136218) (width 1) (layer F.Cu) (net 6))
 (segment (start 49 121.737259) (end 54.398959 127.136218) (width 1) (layer F.Cu) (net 6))
 (segment (start 88.23 123.23) (end 92 119.46) (width 1) (layer F.Cu) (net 6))
 (segment (start 87.95 123.23) (end 88.23 123.23) (width 1) (layer F.Cu) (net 6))
 (segment (start 91 113.095) (end 89.15 113.095) (width 1) (layer F.Cu) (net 6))
 (segment (start 92 114.095) (end 91 113.095) (width 1) (layer F.Cu) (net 6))
 (segment (start 92 119.46) (end 92 114.095) (width 1) (layer F.Cu) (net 6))
 (segment (start 89.15 106.65) (end 89 106.5) (width 1) (layer F.Cu) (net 6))
 (segment (start 89.15 113.095) (end 89.15 106.65) (width 1) (layer F.Cu) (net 6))
 (segment (start 103.141041 130.601041) (end 92 119.46) (width 1) (layer F.Cu) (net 6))
 (segment (start 122.136218 130.601041) (end 103.141041 130.601041) (width 1) (layer F.Cu) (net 6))
 (segment (start 75.5 102.5) (end 51.969998 102.5) (width 1) (layer F.Cu) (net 6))
 (segment (start 87 91) (end 75.5 102.5) (width 1) (layer F.Cu) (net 6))
 (segment (start 94 91) (end 87 91) (width 1) (layer F.Cu) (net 6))
 (segment (start 95 92) (end 94 91) (width 1) (layer F.Cu) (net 6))
 (segment (start 95 100.5) (end 95 92) (width 1) (layer F.Cu) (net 6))
 (segment (start 89 106.5) (end 95 100.5) (width 1) (layer F.Cu) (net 6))
 (segment (start 49 121.737259) (end 49 105.469998) (width 1) (layer F.Cu) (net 6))
 (segment (start 52.25 92.25) (end 49.93 92.25) (width 1) (layer F.Cu) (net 6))
 (segment (start 57.863782 86.636218) (end 52.25 92.25) (width 1) (layer F.Cu) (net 6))
 (segment (start 49.93 92.25) (end 49.75 92.25) (width 1) (layer F.Cu) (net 6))
 (segment (start 49 105.469998) (end 51.969998 102.5) (width 1) (layer F.Cu) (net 6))
 (segment (start 54.398959 130.398959) (end 54.398959 127.136218) (width 1) (layer F.Cu) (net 6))
 (segment (start 52.5 134.5) (end 52.5 132.297918) (width 1) (layer F.Cu) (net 6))
 (segment (start 52.5 132.297918) (end 54.398959 130.398959) (width 1) (layer F.Cu) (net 6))
 (segment (start 54.5 136.5) (end 52.5 134.5) (width 1) (layer F.Cu) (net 6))
 (segment (start 97.242082 136.5) (end 54.5 136.5) (width 1) (layer F.Cu) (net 6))
 (segment (start 103.141041 130.601041) (end 97.242082 136.5) (width 1) (layer F.Cu) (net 6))
 (segment (start 57.863782 59.398959) (end 53.898959 59.398959) (width 1) (layer F.Cu) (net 6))
 (segment (start 53.898959 59.398959) (end 53 58.5) (width 1) (layer F.Cu) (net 6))
 (segment (start 53 58.5) (end 48 58.5) (width 1) (layer F.Cu) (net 6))
 (segment (start 48 58.5) (end 46 60.5) (width 1) (layer F.Cu) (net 6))
 (segment (start 45.969999 81.530001) (end 45.969999 99.469999) (width 1) (layer F.Cu) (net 6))
 (segment (start 46 81.5) (end 45.969999 81.530001) (width 1) (layer F.Cu) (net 6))
 (segment (start 46 60.5) (end 46 81.5) (width 1) (layer F.Cu) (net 6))
 (segment (start 45.969999 99.469999) (end 46 99.5) (width 1) (layer F.Cu) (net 6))
 (segment (start 46 125.797918) (end 52.5 132.297918) (width 1) (layer F.Cu) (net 6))
 (segment (start 46 99.5) (end 46 125.797918) (width 1) (layer F.Cu) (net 6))
 (segment (start 57.863782 59.398959) (end 57.863782 86.636218) (width 1) (layer F.Cu) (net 6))
 (segment (start 57.863782 59.398959) (end 93.898959 59.398959) (width 1) (layer F.Cu) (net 6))
 (segment (start 123.964823 64.5) (end 125.601041 62.863782) (width 1) (layer F.Cu) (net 6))
 (segment (start 99 64.5) (end 123.964823 64.5) (width 1) (layer F.Cu) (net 6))
 (segment (start 93.898959 59.398959) (end 99 64.5) (width 1) (layer F.Cu) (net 6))
 (segment (start 86 120.055) (end 89.15 116.905) (width 0.5) (layer F.Cu) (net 8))
 (segment (start 86 124) (end 86 120.055) (width 0.5) (layer F.Cu) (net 8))
 (segment (start 86.5 124.5) (end 86 124) (width 0.5) (layer F.Cu) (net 8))
 (segment (start 87.95 124.5) (end 86.5 124.5) (width 0.5) (layer F.Cu) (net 8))
 (segment (start 82.898959 130.601041) (end 57.863782 130.601041) (width 0.5) (layer F.Cu) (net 8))
 (segment (start 86 127.5) (end 82.898959 130.601041) (width 0.5) (layer F.Cu) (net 8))
 (segment (start 86 125.339998) (end 86 127.5) (width 0.5) (layer F.Cu) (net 8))
 (segment (start 86.839998 124.5) (end 86 125.339998) (width 0.5) (layer F.Cu) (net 8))
 (segment (start 87.95 124.5) (end 86.839998 124.5) (width 0.5) (layer F.Cu) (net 8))
 (segment (start 87.8 115.635) (end 89.15 115.635) (width 0.5) (layer F.Cu) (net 5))
 (segment (start 84.05 119.385) (end 87.8 115.635) (width 0.5) (layer F.Cu) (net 5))
 (segment (start 84.05 123.23) (end 84.05 119.385) (width 0.5) (layer F.Cu) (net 5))
 (segment (start 82 124.5) (end 84.05 124.5) (width 0.5) (layer F.Cu) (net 7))
 (segment (start 81 123.5) (end 82 124.5) (width 0.5) (layer F.Cu) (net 7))
 (segment (start 81 121.165) (end 81 123.5) (width 0.5) (layer F.Cu) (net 7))
 (segment (start 87.8 114.365) (end 81 121.165) (width 0.5) (layer F.Cu) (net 7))
 (segment (start 89.15 114.365) (end 87.8 114.365) (width 0.5) (layer F.Cu) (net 7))
 (segment (start 78.905 113.095) (end 81.85 113.095) (width 0.5) (layer F.Cu) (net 9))
 (segment (start 76.5 115.5) (end 78.905 113.095) (width 0.5) (layer F.Cu) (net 9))
 (segment (start 76.5 124.5) (end 76.5 115.5) (width 0.5) (layer F.Cu) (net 9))
 (segment (start 77.77 125.77) (end 76.5 124.5) (width 0.5) (layer F.Cu) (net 9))
 (segment (start 84.05 125.77) (end 77.77 125.77) (width 0.5) (layer F.Cu) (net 9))
 (segment (start 115.880001 97.194999) (end 114.075 99) (width 0.5) (layer F.Cu) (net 10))
 (segment (start 115.880001 93.260002) (end 115.880001 97.194999) (width 0.5) (layer F.Cu) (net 10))
 (segment (start 115.669999 93.05) (end 115.880001 93.260002) (width 0.5) (layer F.Cu) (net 10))
 (segment (start 114.9 93.05) (end 115.669999 93.05) (width 0.5) (layer F.Cu) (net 10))
 (segment (start 117.1 88.1) (end 117 88) (width 0.5) (layer F.Cu) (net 11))
 (segment (start 117.1 93.05) (end 117.1 88.1) (width 0.5) (layer F.Cu) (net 11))
 (segment (start 90 102.575) (end 89 103.575) (width 0.5) (layer F.Cu) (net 12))
 (segment (start 90 96.925) (end 90 102.575) (width 0.5) (layer F.Cu) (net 12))
 (segment (start 83.2 114.365) (end 81.85 114.365) (width 0.5) (layer F.Cu) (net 12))
 (segment (start 89 103.575) (end 87.425 103.575) (width 0.5) (layer F.Cu) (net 12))
 (segment (start 87.425 103.575) (end 84.75 106.25) (width 0.5) (layer F.Cu) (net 12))
 (segment (start 84.75 112.815) (end 83.2 114.365) (width 0.5) (layer F.Cu) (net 12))
 (segment (start 84.75 106.25) (end 84.75 112.815) (width 0.5) (layer F.Cu) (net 12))
 (segment (start 47.5 124.762741) (end 52.136218 129.398959) (width 0.5) (layer F.Cu) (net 14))
 (segment (start 47.5 104.5) (end 47.5 124.762741) (width 0.5) (layer F.Cu) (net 14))
 (segment (start 48 104) (end 47.5 104.5) (width 0.5) (layer F.Cu) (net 14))
 (segment (start 48 97.162002) (end 48 104) (width 0.5) (layer F.Cu) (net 14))
 (segment (start 47.269999 92.567999) (end 47.269999 96.432001) (width 0.5) (layer F.Cu) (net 14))
 (segment (start 47.269999 96.432001) (end 48 97.162002) (width 0.5) (layer F.Cu) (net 14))
 (segment (start 48.429999 91.407999) (end 47.269999 92.567999) (width 0.5) (layer F.Cu) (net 14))
 (segment (start 48.429999 68.832742) (end 48.429999 91.407999) (width 0.5) (layer F.Cu) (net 14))
 (segment (start 54.398959 62.863782) (end 48.429999 68.832742) (width 0.5) (layer F.Cu) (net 14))
 (segment (start 55.601041 57.136218) (end 59.5 53.237259) (width 0.5) (layer F.Cu) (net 15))
 (segment (start 115.974518 53.237259) (end 122.136218 59.398959) (width 0.5) (layer F.Cu) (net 15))
 (segment (start 59.5 53.237259) (end 115.974518 53.237259) (width 0.5) (layer F.Cu) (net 15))
 (segment (start 134 66.737259) (end 127.863782 60.601041) (width 0.5) (layer F.Cu) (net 16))
 (segment (start 134 118.737259) (end 134 66.737259) (width 0.5) (layer F.Cu) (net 16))
 (segment (start 125.601041 127.136218) (end 134 118.737259) (width 0.5) (layer F.Cu) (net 16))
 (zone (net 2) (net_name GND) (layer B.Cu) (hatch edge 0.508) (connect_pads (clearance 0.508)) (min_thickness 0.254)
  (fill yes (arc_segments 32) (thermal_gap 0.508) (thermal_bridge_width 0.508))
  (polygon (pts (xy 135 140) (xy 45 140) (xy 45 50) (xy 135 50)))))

